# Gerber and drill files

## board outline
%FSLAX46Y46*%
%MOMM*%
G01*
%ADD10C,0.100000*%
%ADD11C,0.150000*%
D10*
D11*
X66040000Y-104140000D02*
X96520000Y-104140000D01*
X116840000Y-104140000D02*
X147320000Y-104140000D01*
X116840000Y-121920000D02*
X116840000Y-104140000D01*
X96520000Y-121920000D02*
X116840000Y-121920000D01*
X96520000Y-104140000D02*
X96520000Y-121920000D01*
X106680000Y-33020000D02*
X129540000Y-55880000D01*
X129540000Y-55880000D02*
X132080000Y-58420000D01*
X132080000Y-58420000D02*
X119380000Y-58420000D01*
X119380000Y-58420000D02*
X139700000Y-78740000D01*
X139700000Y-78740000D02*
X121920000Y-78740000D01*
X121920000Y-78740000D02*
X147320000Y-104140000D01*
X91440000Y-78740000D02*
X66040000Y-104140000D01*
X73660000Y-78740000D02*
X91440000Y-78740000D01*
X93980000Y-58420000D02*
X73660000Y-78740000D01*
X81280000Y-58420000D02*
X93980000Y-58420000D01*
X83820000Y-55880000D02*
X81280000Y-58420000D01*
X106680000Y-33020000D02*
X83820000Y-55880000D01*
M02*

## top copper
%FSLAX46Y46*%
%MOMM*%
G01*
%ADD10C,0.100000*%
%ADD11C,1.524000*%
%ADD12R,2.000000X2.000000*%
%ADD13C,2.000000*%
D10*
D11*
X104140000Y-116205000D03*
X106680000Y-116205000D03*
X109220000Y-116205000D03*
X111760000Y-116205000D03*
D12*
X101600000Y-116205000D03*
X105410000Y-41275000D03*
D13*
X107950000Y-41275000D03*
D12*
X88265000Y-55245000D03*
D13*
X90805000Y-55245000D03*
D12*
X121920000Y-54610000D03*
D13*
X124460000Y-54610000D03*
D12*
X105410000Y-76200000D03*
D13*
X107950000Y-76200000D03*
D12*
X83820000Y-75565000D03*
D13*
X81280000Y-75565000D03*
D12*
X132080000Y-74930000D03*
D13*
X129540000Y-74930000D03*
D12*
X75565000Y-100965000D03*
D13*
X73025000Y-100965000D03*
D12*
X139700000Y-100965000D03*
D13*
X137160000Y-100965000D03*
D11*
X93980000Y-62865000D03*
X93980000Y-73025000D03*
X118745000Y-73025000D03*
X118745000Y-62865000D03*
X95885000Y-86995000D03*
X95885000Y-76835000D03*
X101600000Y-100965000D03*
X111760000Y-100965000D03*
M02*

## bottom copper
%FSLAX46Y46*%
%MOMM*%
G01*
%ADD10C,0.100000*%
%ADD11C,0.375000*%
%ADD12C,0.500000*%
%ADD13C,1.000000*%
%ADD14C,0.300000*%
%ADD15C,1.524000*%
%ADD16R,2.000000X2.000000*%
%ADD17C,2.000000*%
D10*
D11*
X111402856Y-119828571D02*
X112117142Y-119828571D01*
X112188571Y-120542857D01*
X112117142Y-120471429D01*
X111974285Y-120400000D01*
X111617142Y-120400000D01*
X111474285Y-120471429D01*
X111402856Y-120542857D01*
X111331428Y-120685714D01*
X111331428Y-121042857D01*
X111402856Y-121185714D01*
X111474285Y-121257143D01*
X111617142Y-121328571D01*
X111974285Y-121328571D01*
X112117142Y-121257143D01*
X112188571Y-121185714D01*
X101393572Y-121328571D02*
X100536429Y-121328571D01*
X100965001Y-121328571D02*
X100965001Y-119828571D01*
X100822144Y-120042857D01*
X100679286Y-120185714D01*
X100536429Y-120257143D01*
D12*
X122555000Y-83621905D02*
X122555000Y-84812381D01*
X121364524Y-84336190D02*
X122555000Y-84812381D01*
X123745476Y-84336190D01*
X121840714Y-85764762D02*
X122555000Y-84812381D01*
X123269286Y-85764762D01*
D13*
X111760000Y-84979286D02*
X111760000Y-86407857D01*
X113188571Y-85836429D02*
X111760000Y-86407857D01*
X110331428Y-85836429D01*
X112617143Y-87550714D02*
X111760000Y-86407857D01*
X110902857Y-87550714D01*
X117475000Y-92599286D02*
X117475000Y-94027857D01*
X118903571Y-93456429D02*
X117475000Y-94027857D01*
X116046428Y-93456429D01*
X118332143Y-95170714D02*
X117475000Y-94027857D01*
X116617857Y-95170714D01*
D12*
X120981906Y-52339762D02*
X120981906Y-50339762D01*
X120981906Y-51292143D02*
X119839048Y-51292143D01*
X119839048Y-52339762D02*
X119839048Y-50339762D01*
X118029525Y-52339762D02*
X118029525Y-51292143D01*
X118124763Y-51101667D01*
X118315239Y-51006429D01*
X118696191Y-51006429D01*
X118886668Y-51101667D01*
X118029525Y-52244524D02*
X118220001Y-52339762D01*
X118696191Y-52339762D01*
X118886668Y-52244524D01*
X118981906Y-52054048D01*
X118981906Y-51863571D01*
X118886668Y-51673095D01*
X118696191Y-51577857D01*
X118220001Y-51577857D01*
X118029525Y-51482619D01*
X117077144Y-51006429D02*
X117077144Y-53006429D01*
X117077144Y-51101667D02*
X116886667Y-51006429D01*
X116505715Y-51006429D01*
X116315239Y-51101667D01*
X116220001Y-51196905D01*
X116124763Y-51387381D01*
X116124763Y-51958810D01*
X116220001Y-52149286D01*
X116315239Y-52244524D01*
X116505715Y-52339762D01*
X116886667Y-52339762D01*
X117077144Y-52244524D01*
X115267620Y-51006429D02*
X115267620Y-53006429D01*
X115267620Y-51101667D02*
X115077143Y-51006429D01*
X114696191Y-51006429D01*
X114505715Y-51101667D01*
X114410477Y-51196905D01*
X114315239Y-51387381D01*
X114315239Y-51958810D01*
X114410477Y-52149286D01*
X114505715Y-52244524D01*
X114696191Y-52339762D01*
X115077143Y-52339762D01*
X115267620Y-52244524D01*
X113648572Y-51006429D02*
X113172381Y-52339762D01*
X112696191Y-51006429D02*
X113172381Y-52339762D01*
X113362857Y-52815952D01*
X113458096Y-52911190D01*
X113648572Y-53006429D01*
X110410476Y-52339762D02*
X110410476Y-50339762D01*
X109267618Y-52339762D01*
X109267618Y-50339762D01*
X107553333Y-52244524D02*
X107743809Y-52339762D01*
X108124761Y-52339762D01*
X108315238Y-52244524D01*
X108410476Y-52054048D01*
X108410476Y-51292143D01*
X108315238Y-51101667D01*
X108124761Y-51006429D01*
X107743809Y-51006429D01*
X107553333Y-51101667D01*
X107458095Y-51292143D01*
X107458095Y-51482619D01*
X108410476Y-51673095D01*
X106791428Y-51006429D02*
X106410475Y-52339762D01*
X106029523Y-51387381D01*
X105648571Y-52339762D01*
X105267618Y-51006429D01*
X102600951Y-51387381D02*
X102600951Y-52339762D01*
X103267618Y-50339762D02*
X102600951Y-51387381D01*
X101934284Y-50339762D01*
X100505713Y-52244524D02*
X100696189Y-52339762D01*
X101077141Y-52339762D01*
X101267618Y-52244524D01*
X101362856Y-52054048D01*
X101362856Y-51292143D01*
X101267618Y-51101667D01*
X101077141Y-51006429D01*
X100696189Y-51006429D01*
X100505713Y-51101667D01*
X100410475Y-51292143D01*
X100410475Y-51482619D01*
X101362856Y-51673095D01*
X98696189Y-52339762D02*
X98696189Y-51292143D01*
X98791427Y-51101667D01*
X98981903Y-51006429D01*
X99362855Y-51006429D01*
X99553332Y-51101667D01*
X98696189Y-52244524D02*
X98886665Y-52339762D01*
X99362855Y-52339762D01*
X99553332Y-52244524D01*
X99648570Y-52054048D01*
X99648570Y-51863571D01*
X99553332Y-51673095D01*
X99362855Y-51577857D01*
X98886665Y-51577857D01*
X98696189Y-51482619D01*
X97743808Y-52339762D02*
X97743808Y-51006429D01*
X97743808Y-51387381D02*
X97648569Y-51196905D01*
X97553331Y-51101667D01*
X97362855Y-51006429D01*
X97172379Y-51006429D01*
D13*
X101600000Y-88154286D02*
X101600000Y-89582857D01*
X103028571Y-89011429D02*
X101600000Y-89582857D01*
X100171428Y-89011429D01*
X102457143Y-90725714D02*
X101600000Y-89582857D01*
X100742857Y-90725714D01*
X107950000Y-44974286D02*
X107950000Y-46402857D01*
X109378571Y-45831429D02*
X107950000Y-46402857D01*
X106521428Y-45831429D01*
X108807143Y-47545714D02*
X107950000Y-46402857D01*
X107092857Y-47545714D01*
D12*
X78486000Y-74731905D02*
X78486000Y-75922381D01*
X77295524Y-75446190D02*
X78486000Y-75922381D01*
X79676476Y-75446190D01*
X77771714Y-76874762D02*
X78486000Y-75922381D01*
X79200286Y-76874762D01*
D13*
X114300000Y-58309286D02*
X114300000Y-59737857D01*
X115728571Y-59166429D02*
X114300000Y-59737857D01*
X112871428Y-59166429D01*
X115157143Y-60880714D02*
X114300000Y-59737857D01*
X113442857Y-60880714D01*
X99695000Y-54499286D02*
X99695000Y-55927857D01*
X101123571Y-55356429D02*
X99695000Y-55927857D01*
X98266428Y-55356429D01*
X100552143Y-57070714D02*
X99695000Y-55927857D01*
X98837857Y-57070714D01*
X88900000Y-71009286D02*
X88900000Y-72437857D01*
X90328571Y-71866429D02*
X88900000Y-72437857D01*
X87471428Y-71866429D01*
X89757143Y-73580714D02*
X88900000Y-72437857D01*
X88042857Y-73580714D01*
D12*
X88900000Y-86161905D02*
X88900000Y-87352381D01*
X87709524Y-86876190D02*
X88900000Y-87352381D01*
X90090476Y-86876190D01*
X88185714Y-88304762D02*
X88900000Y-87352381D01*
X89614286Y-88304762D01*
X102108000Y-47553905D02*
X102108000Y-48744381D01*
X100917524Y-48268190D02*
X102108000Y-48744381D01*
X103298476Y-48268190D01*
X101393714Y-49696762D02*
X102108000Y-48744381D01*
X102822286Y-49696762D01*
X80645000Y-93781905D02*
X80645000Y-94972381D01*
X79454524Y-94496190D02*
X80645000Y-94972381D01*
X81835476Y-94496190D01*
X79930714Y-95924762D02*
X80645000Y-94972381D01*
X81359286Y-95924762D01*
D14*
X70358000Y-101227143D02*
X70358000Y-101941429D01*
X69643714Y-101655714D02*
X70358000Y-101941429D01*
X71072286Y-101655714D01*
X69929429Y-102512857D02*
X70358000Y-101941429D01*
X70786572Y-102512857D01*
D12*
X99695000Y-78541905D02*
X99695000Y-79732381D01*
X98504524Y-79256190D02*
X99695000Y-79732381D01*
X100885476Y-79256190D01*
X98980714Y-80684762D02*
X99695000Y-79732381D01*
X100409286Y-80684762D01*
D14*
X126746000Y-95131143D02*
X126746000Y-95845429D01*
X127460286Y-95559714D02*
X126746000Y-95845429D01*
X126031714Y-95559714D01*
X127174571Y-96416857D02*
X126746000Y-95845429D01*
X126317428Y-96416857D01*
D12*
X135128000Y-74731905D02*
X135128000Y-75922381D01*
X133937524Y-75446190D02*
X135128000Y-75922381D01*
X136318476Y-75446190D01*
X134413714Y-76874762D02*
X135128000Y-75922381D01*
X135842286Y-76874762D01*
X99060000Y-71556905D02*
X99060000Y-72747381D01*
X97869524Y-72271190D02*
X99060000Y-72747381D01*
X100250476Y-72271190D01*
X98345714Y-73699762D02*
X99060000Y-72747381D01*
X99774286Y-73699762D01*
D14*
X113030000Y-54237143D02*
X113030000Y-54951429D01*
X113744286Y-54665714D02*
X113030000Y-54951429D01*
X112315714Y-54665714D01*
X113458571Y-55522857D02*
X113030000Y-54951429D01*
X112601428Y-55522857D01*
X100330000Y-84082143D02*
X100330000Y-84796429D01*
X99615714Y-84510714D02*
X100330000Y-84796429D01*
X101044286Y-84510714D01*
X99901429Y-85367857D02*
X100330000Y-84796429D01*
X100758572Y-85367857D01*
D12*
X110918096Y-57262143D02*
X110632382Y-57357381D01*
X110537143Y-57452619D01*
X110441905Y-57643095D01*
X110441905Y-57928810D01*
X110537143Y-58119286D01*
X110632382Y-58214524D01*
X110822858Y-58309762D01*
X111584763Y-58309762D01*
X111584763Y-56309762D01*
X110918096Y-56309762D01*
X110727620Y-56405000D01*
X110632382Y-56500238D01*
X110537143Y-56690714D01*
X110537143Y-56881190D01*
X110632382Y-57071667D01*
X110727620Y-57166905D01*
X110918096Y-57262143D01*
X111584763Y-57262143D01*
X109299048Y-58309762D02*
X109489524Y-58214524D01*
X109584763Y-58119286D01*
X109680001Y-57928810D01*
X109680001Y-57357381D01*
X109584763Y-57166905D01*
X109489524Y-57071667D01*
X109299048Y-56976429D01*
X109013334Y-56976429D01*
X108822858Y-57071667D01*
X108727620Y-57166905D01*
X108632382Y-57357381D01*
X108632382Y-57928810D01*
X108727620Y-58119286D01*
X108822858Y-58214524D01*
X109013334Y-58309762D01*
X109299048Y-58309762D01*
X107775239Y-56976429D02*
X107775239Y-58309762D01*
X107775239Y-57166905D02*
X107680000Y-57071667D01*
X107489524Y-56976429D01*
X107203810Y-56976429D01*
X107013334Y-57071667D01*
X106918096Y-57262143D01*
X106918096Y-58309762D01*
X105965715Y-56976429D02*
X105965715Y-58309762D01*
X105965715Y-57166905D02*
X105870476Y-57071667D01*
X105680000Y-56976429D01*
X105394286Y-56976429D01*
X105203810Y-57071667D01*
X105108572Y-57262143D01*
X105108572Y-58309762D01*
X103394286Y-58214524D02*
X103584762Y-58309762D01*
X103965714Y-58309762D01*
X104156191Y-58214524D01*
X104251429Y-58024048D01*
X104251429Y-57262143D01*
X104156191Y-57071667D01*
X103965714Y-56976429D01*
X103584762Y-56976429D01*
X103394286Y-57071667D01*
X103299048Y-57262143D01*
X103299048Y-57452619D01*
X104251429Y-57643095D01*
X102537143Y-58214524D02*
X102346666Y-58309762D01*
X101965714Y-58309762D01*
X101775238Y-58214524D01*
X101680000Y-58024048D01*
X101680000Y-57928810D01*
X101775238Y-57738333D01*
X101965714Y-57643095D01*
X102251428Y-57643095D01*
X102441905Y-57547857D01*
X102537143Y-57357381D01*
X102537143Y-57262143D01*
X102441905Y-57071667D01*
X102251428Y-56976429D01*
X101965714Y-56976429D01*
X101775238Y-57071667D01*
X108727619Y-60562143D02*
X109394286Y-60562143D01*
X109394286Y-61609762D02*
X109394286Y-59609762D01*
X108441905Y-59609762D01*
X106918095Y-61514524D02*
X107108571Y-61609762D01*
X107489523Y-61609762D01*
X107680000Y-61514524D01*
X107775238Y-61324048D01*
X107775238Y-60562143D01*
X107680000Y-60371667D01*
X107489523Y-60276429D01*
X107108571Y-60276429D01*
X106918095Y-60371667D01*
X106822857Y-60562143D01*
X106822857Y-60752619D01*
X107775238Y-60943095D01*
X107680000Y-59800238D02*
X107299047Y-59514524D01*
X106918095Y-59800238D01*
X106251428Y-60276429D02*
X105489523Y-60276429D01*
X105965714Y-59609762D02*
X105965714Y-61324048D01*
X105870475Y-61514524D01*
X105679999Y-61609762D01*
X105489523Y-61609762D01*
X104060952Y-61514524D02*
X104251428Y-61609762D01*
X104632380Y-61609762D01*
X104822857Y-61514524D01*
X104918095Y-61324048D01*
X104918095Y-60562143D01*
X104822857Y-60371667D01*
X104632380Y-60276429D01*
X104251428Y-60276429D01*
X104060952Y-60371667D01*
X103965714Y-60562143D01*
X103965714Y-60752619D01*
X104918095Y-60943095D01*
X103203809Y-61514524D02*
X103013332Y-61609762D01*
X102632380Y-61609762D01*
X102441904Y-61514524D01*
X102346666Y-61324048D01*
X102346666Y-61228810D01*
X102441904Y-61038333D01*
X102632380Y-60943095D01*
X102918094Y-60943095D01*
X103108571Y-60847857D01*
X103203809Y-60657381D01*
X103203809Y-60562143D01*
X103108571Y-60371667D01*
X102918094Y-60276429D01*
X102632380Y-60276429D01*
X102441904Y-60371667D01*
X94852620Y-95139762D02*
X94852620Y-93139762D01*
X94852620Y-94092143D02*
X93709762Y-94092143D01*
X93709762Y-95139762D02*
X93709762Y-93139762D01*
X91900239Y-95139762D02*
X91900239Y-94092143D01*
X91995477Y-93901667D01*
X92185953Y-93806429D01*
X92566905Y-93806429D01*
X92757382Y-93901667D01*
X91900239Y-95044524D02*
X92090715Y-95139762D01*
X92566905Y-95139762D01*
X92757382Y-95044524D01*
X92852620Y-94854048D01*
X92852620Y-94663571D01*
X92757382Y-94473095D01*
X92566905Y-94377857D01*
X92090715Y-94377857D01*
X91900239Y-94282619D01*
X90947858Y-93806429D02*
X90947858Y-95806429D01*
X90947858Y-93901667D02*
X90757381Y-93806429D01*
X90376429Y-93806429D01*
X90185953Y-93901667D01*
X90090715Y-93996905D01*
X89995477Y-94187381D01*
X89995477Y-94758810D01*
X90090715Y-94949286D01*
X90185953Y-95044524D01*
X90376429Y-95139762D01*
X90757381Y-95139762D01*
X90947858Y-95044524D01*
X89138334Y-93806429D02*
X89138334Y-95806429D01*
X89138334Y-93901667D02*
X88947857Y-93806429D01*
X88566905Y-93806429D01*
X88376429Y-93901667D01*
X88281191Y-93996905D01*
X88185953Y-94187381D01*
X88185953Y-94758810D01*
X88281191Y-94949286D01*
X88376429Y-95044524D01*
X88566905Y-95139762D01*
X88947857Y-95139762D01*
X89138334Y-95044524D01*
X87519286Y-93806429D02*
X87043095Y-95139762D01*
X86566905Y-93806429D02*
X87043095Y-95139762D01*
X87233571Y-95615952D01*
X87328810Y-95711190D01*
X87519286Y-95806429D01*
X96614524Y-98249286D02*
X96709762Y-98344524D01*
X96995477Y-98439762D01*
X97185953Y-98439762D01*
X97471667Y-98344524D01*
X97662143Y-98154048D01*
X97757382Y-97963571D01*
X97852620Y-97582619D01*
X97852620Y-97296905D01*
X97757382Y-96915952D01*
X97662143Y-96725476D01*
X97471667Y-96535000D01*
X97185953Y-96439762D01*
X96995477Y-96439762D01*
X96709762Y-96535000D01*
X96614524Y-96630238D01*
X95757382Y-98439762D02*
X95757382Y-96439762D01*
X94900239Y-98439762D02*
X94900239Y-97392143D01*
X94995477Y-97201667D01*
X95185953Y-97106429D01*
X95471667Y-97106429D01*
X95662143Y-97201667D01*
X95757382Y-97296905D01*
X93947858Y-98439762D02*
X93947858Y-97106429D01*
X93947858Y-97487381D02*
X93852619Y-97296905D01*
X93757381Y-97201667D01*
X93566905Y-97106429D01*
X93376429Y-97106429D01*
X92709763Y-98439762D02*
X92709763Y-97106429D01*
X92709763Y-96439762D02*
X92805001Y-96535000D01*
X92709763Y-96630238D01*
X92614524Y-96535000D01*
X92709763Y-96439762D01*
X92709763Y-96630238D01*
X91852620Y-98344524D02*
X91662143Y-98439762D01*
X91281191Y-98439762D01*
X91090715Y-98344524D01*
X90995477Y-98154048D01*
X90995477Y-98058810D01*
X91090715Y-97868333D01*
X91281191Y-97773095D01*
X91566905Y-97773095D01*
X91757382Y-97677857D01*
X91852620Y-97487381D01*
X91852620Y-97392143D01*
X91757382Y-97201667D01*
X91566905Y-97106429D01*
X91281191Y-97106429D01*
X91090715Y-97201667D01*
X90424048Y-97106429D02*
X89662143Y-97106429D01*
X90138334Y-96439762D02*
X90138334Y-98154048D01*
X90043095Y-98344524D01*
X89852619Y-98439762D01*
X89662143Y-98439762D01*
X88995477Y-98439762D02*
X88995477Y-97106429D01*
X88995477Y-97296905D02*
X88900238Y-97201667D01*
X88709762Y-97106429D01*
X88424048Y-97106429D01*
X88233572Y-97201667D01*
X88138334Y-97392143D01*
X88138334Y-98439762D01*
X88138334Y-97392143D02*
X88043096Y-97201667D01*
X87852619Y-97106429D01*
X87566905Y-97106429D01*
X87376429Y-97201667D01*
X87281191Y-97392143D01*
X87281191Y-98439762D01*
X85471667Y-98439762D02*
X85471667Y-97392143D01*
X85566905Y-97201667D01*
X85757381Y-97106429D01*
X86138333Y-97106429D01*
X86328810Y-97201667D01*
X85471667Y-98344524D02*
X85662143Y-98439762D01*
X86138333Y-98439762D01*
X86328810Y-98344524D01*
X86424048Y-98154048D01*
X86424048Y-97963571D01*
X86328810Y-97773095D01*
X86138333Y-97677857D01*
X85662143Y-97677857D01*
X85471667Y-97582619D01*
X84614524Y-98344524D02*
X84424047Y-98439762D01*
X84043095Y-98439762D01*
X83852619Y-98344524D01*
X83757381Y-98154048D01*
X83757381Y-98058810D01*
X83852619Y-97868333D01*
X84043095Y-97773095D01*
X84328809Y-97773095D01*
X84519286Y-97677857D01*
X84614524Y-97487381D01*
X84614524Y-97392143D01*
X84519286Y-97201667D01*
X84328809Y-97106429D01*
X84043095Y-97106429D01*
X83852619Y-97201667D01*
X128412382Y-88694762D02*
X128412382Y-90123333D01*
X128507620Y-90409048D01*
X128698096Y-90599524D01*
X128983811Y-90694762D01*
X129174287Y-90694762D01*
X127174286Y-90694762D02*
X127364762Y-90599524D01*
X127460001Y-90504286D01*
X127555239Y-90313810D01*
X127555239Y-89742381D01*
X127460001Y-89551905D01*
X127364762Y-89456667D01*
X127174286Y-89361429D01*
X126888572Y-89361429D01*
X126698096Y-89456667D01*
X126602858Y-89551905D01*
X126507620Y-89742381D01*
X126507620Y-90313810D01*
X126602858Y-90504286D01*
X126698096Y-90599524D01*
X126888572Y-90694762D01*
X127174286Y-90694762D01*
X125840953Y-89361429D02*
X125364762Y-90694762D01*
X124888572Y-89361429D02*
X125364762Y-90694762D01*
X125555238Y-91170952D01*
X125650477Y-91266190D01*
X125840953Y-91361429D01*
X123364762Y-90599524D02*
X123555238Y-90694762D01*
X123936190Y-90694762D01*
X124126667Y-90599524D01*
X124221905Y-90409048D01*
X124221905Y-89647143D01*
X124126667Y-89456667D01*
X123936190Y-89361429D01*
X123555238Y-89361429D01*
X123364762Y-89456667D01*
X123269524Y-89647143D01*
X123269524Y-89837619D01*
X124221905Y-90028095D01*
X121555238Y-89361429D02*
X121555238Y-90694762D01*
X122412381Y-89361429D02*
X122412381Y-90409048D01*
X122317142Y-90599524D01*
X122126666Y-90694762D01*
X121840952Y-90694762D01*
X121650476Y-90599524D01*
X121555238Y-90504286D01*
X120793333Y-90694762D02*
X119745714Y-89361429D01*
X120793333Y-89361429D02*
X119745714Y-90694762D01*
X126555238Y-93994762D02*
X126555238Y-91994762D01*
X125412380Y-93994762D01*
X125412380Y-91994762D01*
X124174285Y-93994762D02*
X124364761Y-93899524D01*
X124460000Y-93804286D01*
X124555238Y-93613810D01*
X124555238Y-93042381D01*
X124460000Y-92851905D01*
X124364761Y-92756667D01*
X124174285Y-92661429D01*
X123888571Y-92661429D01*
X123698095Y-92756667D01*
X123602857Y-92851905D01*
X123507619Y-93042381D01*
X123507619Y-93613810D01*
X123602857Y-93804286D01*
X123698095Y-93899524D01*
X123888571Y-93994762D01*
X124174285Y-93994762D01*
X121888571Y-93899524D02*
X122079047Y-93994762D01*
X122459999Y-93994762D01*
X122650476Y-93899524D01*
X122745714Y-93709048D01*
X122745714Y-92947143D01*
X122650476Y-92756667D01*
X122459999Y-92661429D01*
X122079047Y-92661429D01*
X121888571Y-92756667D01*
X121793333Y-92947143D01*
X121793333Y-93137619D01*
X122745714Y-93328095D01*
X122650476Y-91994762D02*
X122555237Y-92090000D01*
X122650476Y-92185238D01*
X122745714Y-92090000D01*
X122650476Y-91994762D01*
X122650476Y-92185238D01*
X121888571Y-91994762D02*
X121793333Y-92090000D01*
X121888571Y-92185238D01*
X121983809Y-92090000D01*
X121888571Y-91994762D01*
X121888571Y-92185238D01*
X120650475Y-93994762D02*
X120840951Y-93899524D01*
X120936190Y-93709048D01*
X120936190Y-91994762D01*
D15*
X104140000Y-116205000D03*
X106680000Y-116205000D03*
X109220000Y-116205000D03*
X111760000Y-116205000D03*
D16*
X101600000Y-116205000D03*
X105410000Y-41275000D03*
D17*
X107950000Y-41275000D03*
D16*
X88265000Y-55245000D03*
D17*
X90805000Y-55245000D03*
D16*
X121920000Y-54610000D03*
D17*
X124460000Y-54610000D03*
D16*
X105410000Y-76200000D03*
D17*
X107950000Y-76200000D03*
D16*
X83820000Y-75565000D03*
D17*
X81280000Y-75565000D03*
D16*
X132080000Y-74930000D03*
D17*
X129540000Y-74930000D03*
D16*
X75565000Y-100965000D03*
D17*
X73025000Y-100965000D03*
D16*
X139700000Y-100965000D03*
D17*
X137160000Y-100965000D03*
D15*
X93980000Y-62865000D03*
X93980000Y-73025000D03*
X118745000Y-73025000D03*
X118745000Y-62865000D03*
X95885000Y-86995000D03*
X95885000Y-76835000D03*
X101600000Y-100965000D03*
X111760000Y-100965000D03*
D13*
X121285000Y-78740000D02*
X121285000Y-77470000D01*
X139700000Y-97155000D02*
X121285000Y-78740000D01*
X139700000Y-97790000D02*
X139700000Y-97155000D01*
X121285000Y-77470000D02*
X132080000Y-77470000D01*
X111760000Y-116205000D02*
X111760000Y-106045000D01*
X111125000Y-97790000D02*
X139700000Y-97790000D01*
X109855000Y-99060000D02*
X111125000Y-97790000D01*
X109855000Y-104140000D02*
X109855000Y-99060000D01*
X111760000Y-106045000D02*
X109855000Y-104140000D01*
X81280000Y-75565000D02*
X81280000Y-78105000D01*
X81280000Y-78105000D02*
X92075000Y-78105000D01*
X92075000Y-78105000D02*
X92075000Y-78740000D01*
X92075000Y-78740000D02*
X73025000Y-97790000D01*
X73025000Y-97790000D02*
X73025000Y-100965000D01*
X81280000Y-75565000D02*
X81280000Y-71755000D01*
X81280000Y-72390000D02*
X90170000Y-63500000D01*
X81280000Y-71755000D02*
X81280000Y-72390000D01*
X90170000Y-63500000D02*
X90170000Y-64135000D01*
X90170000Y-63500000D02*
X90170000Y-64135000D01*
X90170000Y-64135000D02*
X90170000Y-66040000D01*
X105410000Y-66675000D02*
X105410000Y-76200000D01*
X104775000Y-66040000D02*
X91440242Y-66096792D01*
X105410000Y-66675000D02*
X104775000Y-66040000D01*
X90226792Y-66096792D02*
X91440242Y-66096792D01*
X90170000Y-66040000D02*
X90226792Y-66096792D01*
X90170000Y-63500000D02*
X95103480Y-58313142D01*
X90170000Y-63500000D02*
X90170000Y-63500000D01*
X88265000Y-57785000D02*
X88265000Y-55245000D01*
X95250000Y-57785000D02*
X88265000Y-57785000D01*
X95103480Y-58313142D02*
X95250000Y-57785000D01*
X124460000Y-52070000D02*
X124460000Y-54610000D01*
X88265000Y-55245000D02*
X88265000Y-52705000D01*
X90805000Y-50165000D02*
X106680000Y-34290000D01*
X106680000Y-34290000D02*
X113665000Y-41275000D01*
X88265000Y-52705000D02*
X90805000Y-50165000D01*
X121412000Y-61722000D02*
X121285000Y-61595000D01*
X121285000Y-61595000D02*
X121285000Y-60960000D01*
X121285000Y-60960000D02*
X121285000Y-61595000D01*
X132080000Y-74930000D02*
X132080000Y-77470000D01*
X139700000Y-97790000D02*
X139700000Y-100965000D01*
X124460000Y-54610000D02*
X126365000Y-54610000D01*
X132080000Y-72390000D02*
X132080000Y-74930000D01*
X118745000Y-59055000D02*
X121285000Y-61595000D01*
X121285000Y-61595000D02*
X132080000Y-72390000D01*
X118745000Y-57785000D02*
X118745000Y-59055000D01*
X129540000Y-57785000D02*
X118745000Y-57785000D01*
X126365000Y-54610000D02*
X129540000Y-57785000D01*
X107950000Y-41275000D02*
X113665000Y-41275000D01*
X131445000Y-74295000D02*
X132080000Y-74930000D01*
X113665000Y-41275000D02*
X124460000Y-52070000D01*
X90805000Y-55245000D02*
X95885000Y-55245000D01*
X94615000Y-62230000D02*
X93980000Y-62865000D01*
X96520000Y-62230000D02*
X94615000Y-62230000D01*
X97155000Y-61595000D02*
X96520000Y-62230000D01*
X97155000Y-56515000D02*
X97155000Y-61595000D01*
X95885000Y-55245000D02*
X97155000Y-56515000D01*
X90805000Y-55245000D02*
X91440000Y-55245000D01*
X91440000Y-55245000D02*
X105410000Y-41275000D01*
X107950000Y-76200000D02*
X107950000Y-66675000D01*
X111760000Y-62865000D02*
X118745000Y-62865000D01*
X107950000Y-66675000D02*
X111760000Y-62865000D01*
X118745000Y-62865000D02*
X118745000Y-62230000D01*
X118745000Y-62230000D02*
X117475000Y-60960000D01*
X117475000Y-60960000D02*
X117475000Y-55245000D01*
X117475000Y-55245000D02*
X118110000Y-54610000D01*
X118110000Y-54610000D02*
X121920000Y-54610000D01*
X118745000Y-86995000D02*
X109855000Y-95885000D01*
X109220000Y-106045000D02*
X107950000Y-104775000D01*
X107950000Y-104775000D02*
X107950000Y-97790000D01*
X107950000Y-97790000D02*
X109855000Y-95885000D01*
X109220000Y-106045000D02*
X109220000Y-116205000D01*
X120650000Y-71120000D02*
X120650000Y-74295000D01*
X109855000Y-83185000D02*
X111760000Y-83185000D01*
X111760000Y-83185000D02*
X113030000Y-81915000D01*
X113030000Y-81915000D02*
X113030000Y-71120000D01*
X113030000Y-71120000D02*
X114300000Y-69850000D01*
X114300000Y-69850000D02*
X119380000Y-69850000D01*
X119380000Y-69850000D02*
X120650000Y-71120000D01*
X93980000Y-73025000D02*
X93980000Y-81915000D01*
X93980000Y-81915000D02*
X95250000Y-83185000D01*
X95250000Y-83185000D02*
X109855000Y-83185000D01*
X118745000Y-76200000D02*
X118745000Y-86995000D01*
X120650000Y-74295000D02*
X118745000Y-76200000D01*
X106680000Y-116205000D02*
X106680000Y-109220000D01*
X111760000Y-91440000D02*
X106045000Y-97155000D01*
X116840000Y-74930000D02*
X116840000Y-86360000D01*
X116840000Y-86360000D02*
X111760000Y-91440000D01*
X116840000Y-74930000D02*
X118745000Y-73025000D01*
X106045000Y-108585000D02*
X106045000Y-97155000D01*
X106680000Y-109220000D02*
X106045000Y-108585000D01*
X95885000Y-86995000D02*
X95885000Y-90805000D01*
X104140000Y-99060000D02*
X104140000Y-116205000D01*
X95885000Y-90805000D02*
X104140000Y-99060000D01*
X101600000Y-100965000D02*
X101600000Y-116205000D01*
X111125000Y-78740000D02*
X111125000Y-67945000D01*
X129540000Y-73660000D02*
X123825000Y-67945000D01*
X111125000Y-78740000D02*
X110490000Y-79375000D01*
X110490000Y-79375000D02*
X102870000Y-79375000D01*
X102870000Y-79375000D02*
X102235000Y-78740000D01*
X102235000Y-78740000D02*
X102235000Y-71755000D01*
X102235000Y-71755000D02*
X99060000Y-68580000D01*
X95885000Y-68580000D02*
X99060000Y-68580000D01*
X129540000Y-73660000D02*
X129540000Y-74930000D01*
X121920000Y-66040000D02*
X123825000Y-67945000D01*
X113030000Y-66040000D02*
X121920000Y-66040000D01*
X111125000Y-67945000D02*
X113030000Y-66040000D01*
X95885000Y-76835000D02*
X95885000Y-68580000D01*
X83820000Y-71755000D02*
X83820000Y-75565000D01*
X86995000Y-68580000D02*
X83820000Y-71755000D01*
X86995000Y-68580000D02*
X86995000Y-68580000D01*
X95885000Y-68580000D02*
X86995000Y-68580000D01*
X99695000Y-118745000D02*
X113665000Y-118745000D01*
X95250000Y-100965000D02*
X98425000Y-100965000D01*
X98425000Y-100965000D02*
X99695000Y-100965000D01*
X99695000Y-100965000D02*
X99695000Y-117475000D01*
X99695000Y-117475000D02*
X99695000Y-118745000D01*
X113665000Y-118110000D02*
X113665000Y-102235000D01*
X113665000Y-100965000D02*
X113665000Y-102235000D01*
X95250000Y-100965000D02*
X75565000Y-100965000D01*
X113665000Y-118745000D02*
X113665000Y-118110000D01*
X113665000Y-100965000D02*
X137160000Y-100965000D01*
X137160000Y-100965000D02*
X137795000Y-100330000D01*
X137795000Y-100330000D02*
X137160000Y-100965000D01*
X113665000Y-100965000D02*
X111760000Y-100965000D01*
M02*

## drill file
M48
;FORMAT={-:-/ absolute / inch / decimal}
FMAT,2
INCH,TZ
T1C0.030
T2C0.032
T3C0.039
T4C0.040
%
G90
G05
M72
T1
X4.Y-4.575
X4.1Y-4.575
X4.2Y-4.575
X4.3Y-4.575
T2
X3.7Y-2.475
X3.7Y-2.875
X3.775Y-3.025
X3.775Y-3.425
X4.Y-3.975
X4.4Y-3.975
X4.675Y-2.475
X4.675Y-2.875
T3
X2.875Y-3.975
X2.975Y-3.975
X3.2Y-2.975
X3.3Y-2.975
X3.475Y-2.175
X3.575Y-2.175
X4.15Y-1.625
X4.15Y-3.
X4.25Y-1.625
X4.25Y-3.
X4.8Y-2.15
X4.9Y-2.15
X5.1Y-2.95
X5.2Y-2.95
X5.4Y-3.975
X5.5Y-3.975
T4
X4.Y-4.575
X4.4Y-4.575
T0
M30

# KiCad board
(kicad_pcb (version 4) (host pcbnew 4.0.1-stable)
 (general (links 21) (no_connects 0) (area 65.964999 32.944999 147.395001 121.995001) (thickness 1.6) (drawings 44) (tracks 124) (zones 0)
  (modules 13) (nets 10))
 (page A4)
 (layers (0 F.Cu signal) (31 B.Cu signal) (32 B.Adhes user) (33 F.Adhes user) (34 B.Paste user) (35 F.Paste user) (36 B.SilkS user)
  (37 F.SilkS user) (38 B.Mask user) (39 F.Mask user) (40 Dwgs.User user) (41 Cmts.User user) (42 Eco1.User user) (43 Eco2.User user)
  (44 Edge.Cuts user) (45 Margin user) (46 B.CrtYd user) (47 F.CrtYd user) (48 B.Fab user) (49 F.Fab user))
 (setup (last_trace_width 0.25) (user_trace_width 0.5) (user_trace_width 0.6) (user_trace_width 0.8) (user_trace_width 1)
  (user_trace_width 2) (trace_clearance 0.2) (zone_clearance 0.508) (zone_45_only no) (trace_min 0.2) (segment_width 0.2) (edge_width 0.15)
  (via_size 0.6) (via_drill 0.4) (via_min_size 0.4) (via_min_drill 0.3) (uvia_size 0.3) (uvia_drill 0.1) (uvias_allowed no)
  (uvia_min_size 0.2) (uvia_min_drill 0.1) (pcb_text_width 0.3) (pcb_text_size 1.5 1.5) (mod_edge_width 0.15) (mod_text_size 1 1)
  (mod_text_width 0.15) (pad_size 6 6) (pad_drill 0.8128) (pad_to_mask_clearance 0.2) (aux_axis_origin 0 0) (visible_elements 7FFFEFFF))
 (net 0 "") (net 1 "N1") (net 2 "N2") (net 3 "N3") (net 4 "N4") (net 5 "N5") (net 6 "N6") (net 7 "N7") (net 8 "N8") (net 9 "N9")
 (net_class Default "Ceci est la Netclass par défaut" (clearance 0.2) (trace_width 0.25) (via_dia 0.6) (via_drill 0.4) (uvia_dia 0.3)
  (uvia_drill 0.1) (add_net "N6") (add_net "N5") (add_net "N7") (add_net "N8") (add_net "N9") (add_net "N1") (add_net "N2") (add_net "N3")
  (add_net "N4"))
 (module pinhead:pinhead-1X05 (layer B.Cu) (at 106.68 116.205)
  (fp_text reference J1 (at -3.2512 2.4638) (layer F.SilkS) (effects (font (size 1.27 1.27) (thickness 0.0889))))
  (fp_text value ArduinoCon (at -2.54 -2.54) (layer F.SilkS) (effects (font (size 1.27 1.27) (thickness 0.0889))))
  (pad 1 thru_hole rect (at -5.08 0) (size 1.524 0) (drill 1.016) (layers *.Cu B.Paste B.SilkS B.Mask) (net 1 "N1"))
  (pad 2 thru_hole circle (at -2.54 0) (size 1.524 1.524) (drill 0.762) (layers *.Cu B.Paste B.SilkS B.Mask) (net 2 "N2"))
  (pad 3 thru_hole circle (at 0 0) (size 1.524 1.524) (drill 0.762) (layers *.Cu B.Paste B.SilkS B.Mask) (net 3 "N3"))
  (pad 4 thru_hole circle (at 2.54 0) (size 1.524 1.524) (drill 0.762) (layers *.Cu B.Paste B.SilkS B.Mask) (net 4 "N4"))
  (pad 5 thru_hole circle (at 5.08 0) (size 1.524 1.524) (drill 1.016) (layers *.Cu *.Mask B.SilkS) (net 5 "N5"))
  (pad 1 thru_hole rect (at -5.08 0) (size 2 2) (drill 0.762) (layers *.Cu *.Mask B.SilkS) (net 1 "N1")))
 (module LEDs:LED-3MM (layer F.Cu) (at 105.41 41.275)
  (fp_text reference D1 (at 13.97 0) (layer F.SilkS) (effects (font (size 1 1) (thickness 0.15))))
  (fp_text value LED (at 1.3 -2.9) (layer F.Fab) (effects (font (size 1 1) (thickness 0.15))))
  (pad 1 thru_hole rect (at 0 0 90) (size 2 2) (drill 1.00076) (layers *.Cu *.Mask F.SilkS) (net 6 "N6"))
  (pad 2 thru_hole circle (at 2.54 0) (size 2 2) (drill 1.00076) (layers *.Cu *.Mask F.SilkS) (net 5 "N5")))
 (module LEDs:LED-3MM (layer F.Cu) (at 88.265 55.245)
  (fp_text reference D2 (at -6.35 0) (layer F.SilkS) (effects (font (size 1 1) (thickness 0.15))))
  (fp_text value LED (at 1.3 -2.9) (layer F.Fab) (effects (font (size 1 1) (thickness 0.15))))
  (pad 1 thru_hole rect (at 0 0 90) (size 2 2) (drill 1.00076) (layers *.Cu *.Mask F.SilkS) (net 5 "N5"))
  (pad 2 thru_hole circle (at 2.54 0) (size 2 2) (drill 1.00076) (layers *.Cu *.Mask F.SilkS) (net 6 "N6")))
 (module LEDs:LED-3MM (layer F.Cu) (at 121.92 54.61)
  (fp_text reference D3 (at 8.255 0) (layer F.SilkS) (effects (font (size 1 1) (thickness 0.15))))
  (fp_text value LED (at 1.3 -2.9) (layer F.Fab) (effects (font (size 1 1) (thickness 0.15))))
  (pad 1 thru_hole rect (at 0 0 90) (size 2 2) (drill 1.00076) (layers *.Cu *.Mask F.SilkS) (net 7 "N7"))
  (pad 2 thru_hole circle (at 2.54 0) (size 2 2) (drill 1.00076) (layers *.Cu *.Mask F.SilkS) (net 5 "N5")))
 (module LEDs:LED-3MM (layer F.Cu) (at 105.41 76.2)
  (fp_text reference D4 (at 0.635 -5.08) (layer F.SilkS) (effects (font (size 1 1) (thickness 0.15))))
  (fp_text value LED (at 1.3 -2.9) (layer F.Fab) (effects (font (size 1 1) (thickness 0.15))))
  (pad 1 thru_hole rect (at 0 0 90) (size 2 2) (drill 1.00076) (layers *.Cu *.Mask F.SilkS) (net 5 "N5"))
  (pad 2 thru_hole circle (at 2.54 0) (size 2 2) (drill 1.00076) (layers *.Cu *.Mask F.SilkS) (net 7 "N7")))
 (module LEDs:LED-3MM (layer F.Cu) (at 83.82 75.565 180)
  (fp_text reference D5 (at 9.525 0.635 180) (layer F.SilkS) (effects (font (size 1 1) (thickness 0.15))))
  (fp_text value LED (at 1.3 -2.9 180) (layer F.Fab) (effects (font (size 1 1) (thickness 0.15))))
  (pad 1 thru_hole rect (at 0 0 270) (size 2 2) (drill 1.00076) (layers *.Cu *.Mask F.SilkS) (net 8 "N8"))
  (pad 2 thru_hole circle (at 2.54 0 180) (size 2 2) (drill 1.00076) (layers *.Cu *.Mask F.SilkS) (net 5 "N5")))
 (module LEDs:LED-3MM (layer F.Cu) (at 132.08 74.93 180)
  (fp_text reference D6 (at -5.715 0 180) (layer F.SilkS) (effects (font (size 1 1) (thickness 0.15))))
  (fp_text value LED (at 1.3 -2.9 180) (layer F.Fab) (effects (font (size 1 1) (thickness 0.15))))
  (pad 1 thru_hole rect (at 0 0 270) (size 2 2) (drill 1.00076) (layers *.Cu *.Mask F.SilkS) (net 5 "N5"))
  (pad 2 thru_hole circle (at 2.54 0 180) (size 2 2) (drill 1.00076) (layers *.Cu *.Mask F.SilkS) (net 8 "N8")))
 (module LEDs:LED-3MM (layer F.Cu) (at 75.565 100.965 180)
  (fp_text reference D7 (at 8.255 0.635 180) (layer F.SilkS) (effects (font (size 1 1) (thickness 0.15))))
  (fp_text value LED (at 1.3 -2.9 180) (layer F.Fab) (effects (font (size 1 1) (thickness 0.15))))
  (pad 1 thru_hole rect (at 0 0 270) (size 2 2) (drill 1.00076) (layers *.Cu *.Mask F.SilkS) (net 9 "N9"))
  (pad 2 thru_hole circle (at 2.54 0 180) (size 2 2) (drill 1.00076) (layers *.Cu *.Mask F.SilkS) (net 5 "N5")))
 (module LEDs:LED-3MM (layer F.Cu) (at 139.7 100.965 180)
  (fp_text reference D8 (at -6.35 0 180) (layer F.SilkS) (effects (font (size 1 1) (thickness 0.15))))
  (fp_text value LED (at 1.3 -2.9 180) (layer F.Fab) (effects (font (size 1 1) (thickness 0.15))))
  (pad 1 thru_hole rect (at 0 0 270) (size 2 2) (drill 1.00076) (layers *.Cu *.Mask F.SilkS) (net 5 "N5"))
  (pad 2 thru_hole circle (at 2.54 0 180) (size 2 2) (drill 1.00076) (layers *.Cu *.Mask F.SilkS) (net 9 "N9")))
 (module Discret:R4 (layer B.Cu) (at 93.98 67.945 270)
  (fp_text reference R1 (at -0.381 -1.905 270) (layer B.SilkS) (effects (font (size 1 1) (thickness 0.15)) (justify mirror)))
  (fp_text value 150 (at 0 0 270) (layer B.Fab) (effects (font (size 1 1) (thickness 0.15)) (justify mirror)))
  (pad 1 thru_hole circle (at -5.08 0 270) (size 1.524 1.524) (drill 0.8128) (layers *.Cu *.Mask B.SilkS) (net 6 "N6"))
  (pad 2 thru_hole circle (at 5.08 0 270) (size 1.524 1.524) (drill 0.8128) (layers *.Cu *.Mask B.SilkS) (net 4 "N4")))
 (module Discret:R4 (layer B.Cu) (at 118.745 67.945 90)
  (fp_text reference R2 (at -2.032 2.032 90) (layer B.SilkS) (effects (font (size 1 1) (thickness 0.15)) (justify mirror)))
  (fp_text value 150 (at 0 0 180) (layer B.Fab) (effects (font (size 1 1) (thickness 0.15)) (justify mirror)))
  (pad 1 thru_hole circle (at -5.08 0 90) (size 1.524 1.524) (drill 0.8128) (layers *.Cu *.Mask B.SilkS) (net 3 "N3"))
  (pad 2 thru_hole circle (at 5.08 0 90) (size 1.524 1.524) (drill 0.8128) (layers *.Cu *.Mask B.SilkS) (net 7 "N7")))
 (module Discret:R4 (layer B.Cu) (at 95.885 81.915 90)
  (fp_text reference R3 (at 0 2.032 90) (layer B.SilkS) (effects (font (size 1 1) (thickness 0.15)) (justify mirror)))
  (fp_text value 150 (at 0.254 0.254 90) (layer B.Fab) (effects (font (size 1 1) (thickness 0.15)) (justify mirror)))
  (pad 1 thru_hole circle (at -5.08 0 90) (size 1.524 1.524) (drill 0.8128) (layers *.Cu *.Mask B.SilkS) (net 2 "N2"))
  (pad 2 thru_hole circle (at 5.08 0 90) (size 1.524 1.524) (drill 0.8128) (layers *.Cu *.Mask B.SilkS) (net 8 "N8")))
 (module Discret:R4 (layer B.Cu) (at 106.68 100.965)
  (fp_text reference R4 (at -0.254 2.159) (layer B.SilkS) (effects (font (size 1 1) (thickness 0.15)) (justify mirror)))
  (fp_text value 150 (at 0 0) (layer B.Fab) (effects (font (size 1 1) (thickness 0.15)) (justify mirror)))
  (pad 1 thru_hole circle (at -5.08 0) (size 1.524 1.524) (drill 0.8128) (layers *.Cu *.Mask B.SilkS) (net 1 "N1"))
  (pad 2 thru_hole circle (at 5.08 0) (size 1.524 1.524) (drill 0.8128) (layers *.Cu *.Mask B.SilkS) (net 9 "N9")))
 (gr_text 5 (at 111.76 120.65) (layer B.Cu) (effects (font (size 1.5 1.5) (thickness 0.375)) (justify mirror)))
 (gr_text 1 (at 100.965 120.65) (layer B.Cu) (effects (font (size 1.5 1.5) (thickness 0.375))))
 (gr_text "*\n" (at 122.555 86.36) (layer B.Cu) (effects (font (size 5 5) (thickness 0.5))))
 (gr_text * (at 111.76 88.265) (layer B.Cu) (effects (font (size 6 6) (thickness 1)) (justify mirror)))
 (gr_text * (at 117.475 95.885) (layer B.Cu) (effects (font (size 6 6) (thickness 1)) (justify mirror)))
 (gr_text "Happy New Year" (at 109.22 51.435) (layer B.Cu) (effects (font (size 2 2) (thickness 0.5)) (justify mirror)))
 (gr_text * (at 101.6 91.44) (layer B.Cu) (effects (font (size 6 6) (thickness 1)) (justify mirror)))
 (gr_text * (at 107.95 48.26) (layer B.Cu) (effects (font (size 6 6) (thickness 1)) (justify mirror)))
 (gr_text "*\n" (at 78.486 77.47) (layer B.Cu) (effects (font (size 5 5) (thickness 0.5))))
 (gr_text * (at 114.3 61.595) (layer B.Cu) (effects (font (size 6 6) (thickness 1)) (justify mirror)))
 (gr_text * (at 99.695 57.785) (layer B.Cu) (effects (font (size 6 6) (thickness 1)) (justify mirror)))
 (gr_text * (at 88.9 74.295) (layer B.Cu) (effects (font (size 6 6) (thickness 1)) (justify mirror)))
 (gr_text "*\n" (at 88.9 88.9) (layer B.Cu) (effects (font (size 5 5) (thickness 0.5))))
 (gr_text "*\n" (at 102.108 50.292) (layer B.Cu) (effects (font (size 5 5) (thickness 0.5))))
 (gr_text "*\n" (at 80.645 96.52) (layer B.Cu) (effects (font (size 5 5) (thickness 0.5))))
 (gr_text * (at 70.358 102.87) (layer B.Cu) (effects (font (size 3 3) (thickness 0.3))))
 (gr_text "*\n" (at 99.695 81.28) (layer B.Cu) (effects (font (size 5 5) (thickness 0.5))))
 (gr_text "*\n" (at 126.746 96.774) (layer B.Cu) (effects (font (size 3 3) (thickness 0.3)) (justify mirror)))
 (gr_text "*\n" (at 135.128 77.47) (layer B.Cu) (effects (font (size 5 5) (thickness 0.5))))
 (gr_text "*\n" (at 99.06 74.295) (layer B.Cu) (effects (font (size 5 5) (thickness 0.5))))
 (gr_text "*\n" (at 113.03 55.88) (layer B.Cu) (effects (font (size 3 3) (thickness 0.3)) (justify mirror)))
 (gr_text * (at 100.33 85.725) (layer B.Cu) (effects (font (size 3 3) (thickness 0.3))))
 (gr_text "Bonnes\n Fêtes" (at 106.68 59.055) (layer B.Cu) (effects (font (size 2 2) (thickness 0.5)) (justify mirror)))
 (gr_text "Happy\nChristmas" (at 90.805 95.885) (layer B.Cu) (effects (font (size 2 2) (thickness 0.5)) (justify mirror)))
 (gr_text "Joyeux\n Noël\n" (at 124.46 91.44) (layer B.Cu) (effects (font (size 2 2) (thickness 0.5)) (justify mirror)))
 (gr_line (start 66.04 104.14) (end 96.52 104.14) (angle 90) (layer Edge.Cuts) (width 0.15))
 (gr_line (start 116.84 104.14) (end 147.32 104.14) (angle 90) (layer Edge.Cuts) (width 0.15))
 (gr_line (start 116.84 121.92) (end 116.84 104.14) (angle 90) (layer Edge.Cuts) (width 0.15))
 (gr_line (start 96.52 121.92) (end 116.84 121.92) (angle 90) (layer Edge.Cuts) (width 0.15))
 (gr_line (start 96.52 104.14) (end 96.52 121.92) (angle 90) (layer Edge.Cuts) (width 0.15))
 (gr_line (start 106.68 33.02) (end 129.54 55.88) (angle 90) (layer Edge.Cuts) (width 0.15))
 (gr_line (start 129.54 55.88) (end 132.08 58.42) (angle 90) (layer Edge.Cuts) (width 0.15))
 (gr_line (start 132.08 58.42) (end 119.38 58.42) (angle 90) (layer Edge.Cuts) (width 0.15))
 (gr_line (start 119.38 58.42) (end 139.7 78.74) (angle 90) (layer Edge.Cuts) (width 0.15))
 (gr_line (start 139.7 78.74) (end 121.92 78.74) (angle 90) (layer Edge.Cuts) (width 0.15))
 (gr_line (start 121.92 78.74) (end 147.32 104.14) (angle 90) (layer Edge.Cuts) (width 0.15))
 (gr_line (start 91.44 78.74) (end 66.04 104.14) (angle 90) (layer Edge.Cuts) (width 0.15))
 (gr_line (start 73.66 78.74) (end 91.44 78.74) (angle 90) (layer Edge.Cuts) (width 0.15))
 (gr_line (start 93.98 58.42) (end 73.66 78.74) (angle 90) (layer Edge.Cuts) (width 0.15))
 (gr_line (start 81.28 58.42) (end 93.98 58.42) (angle 90) (layer Edge.Cuts) (width 0.15))
 (gr_line (start 83.82 55.88) (end 81.28 58.42) (angle 90) (layer Edge.Cuts) (width 0.15))
 (gr_line (start 106.68 33.02) (end 83.82 55.88) (angle 90) (layer Edge.Cuts) (width 0.15))
 (segment (start 121.285 78.74) (end 121.285 77.47) (width 1) (layer B.Cu) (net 5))
 (segment (start 139.7 97.155) (end 121.285 78.74) (width 1) (layer B.Cu) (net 5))
 (segment (start 139.7 97.79) (end 139.7 97.155) (width 1) (layer B.Cu) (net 5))
 (segment (start 121.285 77.47) (end 132.08 77.47) (width 1) (layer B.Cu) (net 5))
 (segment (start 111.76 116.205) (end 111.76 106.045) (width 1) (layer B.Cu) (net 5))
 (segment (start 111.125 97.79) (end 139.7 97.79) (width 1) (layer B.Cu) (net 5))
 (segment (start 109.855 99.06) (end 111.125 97.79) (width 1) (layer B.Cu) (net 5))
 (segment (start 109.855 104.14) (end 109.855 99.06) (width 1) (layer B.Cu) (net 5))
 (segment (start 111.76 106.045) (end 109.855 104.14) (width 1) (layer B.Cu) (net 5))
 (segment (start 81.28 75.565) (end 81.28 78.105) (width 1) (layer B.Cu) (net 5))
 (segment (start 81.28 78.105) (end 92.075 78.105) (width 1) (layer B.Cu) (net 5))
 (segment (start 92.075 78.105) (end 92.075 78.74) (width 1) (layer B.Cu) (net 5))
 (segment (start 92.075 78.74) (end 73.025 97.79) (width 1) (layer B.Cu) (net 5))
 (segment (start 73.025 97.79) (end 73.025 100.965) (width 1) (layer B.Cu) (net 5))
 (segment (start 81.28 75.565) (end 81.28 71.755) (width 1) (layer B.Cu) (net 5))
 (segment (start 81.28 72.39) (end 90.17 63.5) (width 1) (layer B.Cu) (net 5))
 (segment (start 81.28 71.755) (end 81.28 72.39) (width 1) (layer B.Cu) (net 5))
 (segment (start 90.17 63.5) (end 90.17 64.135) (width 1) (layer B.Cu) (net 5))
 (segment (start 90.17 63.5) (end 90.17 64.135) (width 1) (layer B.Cu) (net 5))
 (segment (start 90.17 64.135) (end 90.17 66.04) (width 1) (layer B.Cu) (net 5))
 (segment (start 105.41 66.675) (end 105.41 76.2) (width 1) (layer B.Cu) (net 5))
 (segment (start 104.775 66.04) (end 91.440242 66.096792) (width 1) (layer B.Cu) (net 5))
 (segment (start 105.41 66.675) (end 104.775 66.04) (width 1) (layer B.Cu) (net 5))
 (segment (start 90.226792 66.096792) (end 91.440242 66.096792) (width 1) (layer B.Cu) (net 5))
 (segment (start 90.17 66.04) (end 90.226792 66.096792) (width 1) (layer B.Cu) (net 5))
 (segment (start 90.17 63.5) (end 95.10348 58.313142) (width 1) (layer B.Cu) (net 5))
 (segment (start 90.17 63.5) (end 90.17 63.5) (width 1) (layer B.Cu) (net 5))
 (segment (start 88.265 57.785) (end 88.265 55.245) (width 1) (layer B.Cu) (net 5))
 (segment (start 95.25 57.785) (end 88.265 57.785) (width 1) (layer B.Cu) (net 5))
 (segment (start 95.10348 58.313142) (end 95.25 57.785) (width 1) (layer B.Cu) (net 5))
 (segment (start 124.46 52.07) (end 124.46 54.61) (width 1) (layer B.Cu) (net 5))
 (segment (start 88.265 55.245) (end 88.265 52.705) (width 1) (layer B.Cu) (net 5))
 (segment (start 90.805 50.165) (end 106.68 34.29) (width 1) (layer B.Cu) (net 5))
 (segment (start 106.68 34.29) (end 113.665 41.275) (width 1) (layer B.Cu) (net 5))
 (segment (start 88.265 52.705) (end 90.805 50.165) (width 1) (layer B.Cu) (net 5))
 (segment (start 121.412 61.722) (end 121.285 61.595) (width 1) (layer B.Cu) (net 5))
 (segment (start 121.285 61.595) (end 121.285 60.96) (width 1) (layer B.Cu) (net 5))
 (segment (start 121.285 60.96) (end 121.285 61.595) (width 1) (layer B.Cu) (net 5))
 (segment (start 132.08 74.93) (end 132.08 77.47) (width 1) (layer B.Cu) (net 5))
 (segment (start 139.7 97.79) (end 139.7 100.965) (width 1) (layer B.Cu) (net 5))
 (segment (start 124.46 54.61) (end 126.365 54.61) (width 1) (layer B.Cu) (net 5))
 (segment (start 132.08 72.39) (end 132.08 74.93) (width 1) (layer B.Cu) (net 5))
 (segment (start 118.745 59.055) (end 121.285 61.595) (width 1) (layer B.Cu) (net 5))
 (segment (start 121.285 61.595) (end 132.08 72.39) (width 1) (layer B.Cu) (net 5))
 (segment (start 118.745 57.785) (end 118.745 59.055) (width 1) (layer B.Cu) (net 5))
 (segment (start 129.54 57.785) (end 118.745 57.785) (width 1) (layer B.Cu) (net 5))
 (segment (start 126.365 54.61) (end 129.54 57.785) (width 1) (layer B.Cu) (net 5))
 (segment (start 107.95 41.275) (end 113.665 41.275) (width 1) (layer B.Cu) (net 5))
 (segment (start 131.445 74.295) (end 132.08 74.93) (width 1) (layer B.Cu) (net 5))
 (segment (start 113.665 41.275) (end 124.46 52.07) (width 1) (layer B.Cu) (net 5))
 (segment (start 90.805 55.245) (end 95.885 55.245) (width 1) (layer B.Cu) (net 6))
 (segment (start 94.615 62.23) (end 93.98 62.865) (width 1) (layer B.Cu) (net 6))
 (segment (start 96.52 62.23) (end 94.615 62.23) (width 1) (layer B.Cu) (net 6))
 (segment (start 97.155 61.595) (end 96.52 62.23) (width 1) (layer B.Cu) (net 6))
 (segment (start 97.155 56.515) (end 97.155 61.595) (width 1) (layer B.Cu) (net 6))
 (segment (start 95.885 55.245) (end 97.155 56.515) (width 1) (layer B.Cu) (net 6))
 (segment (start 90.805 55.245) (end 91.44 55.245) (width 1) (layer B.Cu) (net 6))
 (segment (start 91.44 55.245) (end 105.41 41.275) (width 1) (layer B.Cu) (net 6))
 (segment (start 107.95 76.2) (end 107.95 66.675) (width 1) (layer B.Cu) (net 7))
 (segment (start 111.76 62.865) (end 118.745 62.865) (width 1) (layer B.Cu) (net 7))
 (segment (start 107.95 66.675) (end 111.76 62.865) (width 1) (layer B.Cu) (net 7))
 (segment (start 118.745 62.865) (end 118.745 62.23) (width 1) (layer B.Cu) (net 7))
 (segment (start 118.745 62.23) (end 117.475 60.96) (width 1) (layer B.Cu) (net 7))
 (segment (start 117.475 60.96) (end 117.475 55.245) (width 1) (layer B.Cu) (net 7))
 (segment (start 117.475 55.245) (end 118.11 54.61) (width 1) (layer B.Cu) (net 7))
 (segment (start 118.11 54.61) (end 121.92 54.61) (width 1) (layer B.Cu) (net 7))
 (segment (start 118.745 86.995) (end 109.855 95.885) (width 1) (layer B.Cu) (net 4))
 (segment (start 109.22 106.045) (end 107.95 104.775) (width 1) (layer B.Cu) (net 4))
 (segment (start 107.95 104.775) (end 107.95 97.79) (width 1) (layer B.Cu) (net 4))
 (segment (start 107.95 97.79) (end 109.855 95.885) (width 1) (layer B.Cu) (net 4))
 (segment (start 109.22 106.045) (end 109.22 116.205) (width 1) (layer B.Cu) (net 4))
 (segment (start 120.65 71.12) (end 120.65 74.295) (width 1) (layer B.Cu) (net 4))
 (segment (start 109.855 83.185) (end 111.76 83.185) (width 1) (layer B.Cu) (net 4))
 (segment (start 111.76 83.185) (end 113.03 81.915) (width 1) (layer B.Cu) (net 4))
 (segment (start 113.03 81.915) (end 113.03 71.12) (width 1) (layer B.Cu) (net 4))
 (segment (start 113.03 71.12) (end 114.3 69.85) (width 1) (layer B.Cu) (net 4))
 (segment (start 114.3 69.85) (end 119.38 69.85) (width 1) (layer B.Cu) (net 4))
 (segment (start 119.38 69.85) (end 120.65 71.12) (width 1) (layer B.Cu) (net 4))
 (segment (start 93.98 73.025) (end 93.98 81.915) (width 1) (layer B.Cu) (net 4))
 (segment (start 93.98 81.915) (end 95.25 83.185) (width 1) (layer B.Cu) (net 4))
 (segment (start 95.25 83.185) (end 109.855 83.185) (width 1) (layer B.Cu) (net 4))
 (segment (start 118.745 76.2) (end 118.745 86.995) (width 1) (layer B.Cu) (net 4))
 (segment (start 120.65 74.295) (end 118.745 76.2) (width 1) (layer B.Cu) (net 4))
 (segment (start 106.68 116.205) (end 106.68 109.22) (width 1) (layer B.Cu) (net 3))
 (segment (start 111.76 91.44) (end 106.045 97.155) (width 1) (layer B.Cu) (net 3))
 (segment (start 116.84 74.93) (end 116.84 86.36) (width 1) (layer B.Cu) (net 3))
 (segment (start 116.84 86.36) (end 111.76 91.44) (width 1) (layer B.Cu) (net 3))
 (segment (start 116.84 74.93) (end 118.745 73.025) (width 1) (layer B.Cu) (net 3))
 (segment (start 106.045 108.585) (end 106.045 97.155) (width 1) (layer B.Cu) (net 3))
 (segment (start 106.68 109.22) (end 106.045 108.585) (width 1) (layer B.Cu) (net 3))
 (segment (start 95.885 86.995) (end 95.885 90.805) (width 1) (layer B.Cu) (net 2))
 (segment (start 104.14 99.06) (end 104.14 116.205) (width 1) (layer B.Cu) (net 2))
 (segment (start 95.885 90.805) (end 104.14 99.06) (width 1) (layer B.Cu) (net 2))
 (segment (start 101.6 100.965) (end 101.6 116.205) (width 1) (layer B.Cu) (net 1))
 (segment (start 111.125 78.74) (end 111.125 67.945) (width 1) (layer B.Cu) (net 8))
 (segment (start 129.54 73.66) (end 123.825 67.945) (width 1) (layer B.Cu) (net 8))
 (segment (start 111.125 78.74) (end 110.49 79.375) (width 1) (layer B.Cu) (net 8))
 (segment (start 110.49 79.375) (end 102.87 79.375) (width 1) (layer B.Cu) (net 8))
 (segment (start 102.87 79.375) (end 102.235 78.74) (width 1) (layer B.Cu) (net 8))
 (segment (start 102.235 78.74) (end 102.235 71.755) (width 1) (layer B.Cu) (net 8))
 (segment (start 102.235 71.755) (end 99.06 68.58) (width 1) (layer B.Cu) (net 8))
 (segment (start 95.885 68.58) (end 99.06 68.58) (width 1) (layer B.Cu) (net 8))
 (segment (start 129.54 73.66) (end 129.54 74.93) (width 1) (layer B.Cu) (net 8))
 (segment (start 121.92 66.04) (end 123.825 67.945) (width 1) (layer B.Cu) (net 8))
 (segment (start 113.03 66.04) (end 121.92 66.04) (width 1) (layer B.Cu) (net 8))
 (segment (start 111.125 67.945) (end 113.03 66.04) (width 1) (layer B.Cu) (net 8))
 (segment (start 95.885 76.835) (end 95.885 68.58) (width 1) (layer B.Cu) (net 8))
 (segment (start 83.82 71.755) (end 83.82 75.565) (width 1) (layer B.Cu) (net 8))
 (segment (start 86.995 68.58) (end 83.82 71.755) (width 1) (layer B.Cu) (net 8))
 (segment (start 86.995 68.58) (end 86.995 68.58) (width 1) (layer B.Cu) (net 8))
 (segment (start 95.885 68.58) (end 86.995 68.58) (width 1) (layer B.Cu) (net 8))
 (segment (start 99.695 118.745) (end 113.665 118.745) (width 1) (layer B.Cu) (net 9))
 (segment (start 95.25 100.965) (end 98.425 100.965) (width 1) (layer B.Cu) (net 9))
 (segment (start 98.425 100.965) (end 99.695 100.965) (width 1) (layer B.Cu) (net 9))
 (segment (start 99.695 100.965) (end 99.695 117.475) (width 1) (layer B.Cu) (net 9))
 (segment (start 99.695 117.475) (end 99.695 118.745) (width 1) (layer B.Cu) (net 9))
 (segment (start 113.665 118.11) (end 113.665 102.235) (width 1) (layer B.Cu) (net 9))
 (segment (start 113.665 100.965) (end 113.665 102.235) (width 1) (layer B.Cu) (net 9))
 (segment (start 95.25 100.965) (end 75.565 100.965) (width 1) (layer B.Cu) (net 9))
 (segment (start 113.665 118.745) (end 113.665 118.11) (width 1) (layer B.Cu) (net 9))
 (segment (start 113.665 100.965) (end 137.16 100.965) (width 1) (layer B.Cu) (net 9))
 (segment (start 137.16 100.965) (end 137.795 100.33) (width 1) (layer B.Cu) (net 9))
 (segment (start 137.795 100.33) (end 137.16 100.965) (width 1) (layer B.Cu) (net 9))
 (segment (start 113.665 100.965) (end 111.76 100.965) (width 1) (layer B.Cu) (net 9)))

